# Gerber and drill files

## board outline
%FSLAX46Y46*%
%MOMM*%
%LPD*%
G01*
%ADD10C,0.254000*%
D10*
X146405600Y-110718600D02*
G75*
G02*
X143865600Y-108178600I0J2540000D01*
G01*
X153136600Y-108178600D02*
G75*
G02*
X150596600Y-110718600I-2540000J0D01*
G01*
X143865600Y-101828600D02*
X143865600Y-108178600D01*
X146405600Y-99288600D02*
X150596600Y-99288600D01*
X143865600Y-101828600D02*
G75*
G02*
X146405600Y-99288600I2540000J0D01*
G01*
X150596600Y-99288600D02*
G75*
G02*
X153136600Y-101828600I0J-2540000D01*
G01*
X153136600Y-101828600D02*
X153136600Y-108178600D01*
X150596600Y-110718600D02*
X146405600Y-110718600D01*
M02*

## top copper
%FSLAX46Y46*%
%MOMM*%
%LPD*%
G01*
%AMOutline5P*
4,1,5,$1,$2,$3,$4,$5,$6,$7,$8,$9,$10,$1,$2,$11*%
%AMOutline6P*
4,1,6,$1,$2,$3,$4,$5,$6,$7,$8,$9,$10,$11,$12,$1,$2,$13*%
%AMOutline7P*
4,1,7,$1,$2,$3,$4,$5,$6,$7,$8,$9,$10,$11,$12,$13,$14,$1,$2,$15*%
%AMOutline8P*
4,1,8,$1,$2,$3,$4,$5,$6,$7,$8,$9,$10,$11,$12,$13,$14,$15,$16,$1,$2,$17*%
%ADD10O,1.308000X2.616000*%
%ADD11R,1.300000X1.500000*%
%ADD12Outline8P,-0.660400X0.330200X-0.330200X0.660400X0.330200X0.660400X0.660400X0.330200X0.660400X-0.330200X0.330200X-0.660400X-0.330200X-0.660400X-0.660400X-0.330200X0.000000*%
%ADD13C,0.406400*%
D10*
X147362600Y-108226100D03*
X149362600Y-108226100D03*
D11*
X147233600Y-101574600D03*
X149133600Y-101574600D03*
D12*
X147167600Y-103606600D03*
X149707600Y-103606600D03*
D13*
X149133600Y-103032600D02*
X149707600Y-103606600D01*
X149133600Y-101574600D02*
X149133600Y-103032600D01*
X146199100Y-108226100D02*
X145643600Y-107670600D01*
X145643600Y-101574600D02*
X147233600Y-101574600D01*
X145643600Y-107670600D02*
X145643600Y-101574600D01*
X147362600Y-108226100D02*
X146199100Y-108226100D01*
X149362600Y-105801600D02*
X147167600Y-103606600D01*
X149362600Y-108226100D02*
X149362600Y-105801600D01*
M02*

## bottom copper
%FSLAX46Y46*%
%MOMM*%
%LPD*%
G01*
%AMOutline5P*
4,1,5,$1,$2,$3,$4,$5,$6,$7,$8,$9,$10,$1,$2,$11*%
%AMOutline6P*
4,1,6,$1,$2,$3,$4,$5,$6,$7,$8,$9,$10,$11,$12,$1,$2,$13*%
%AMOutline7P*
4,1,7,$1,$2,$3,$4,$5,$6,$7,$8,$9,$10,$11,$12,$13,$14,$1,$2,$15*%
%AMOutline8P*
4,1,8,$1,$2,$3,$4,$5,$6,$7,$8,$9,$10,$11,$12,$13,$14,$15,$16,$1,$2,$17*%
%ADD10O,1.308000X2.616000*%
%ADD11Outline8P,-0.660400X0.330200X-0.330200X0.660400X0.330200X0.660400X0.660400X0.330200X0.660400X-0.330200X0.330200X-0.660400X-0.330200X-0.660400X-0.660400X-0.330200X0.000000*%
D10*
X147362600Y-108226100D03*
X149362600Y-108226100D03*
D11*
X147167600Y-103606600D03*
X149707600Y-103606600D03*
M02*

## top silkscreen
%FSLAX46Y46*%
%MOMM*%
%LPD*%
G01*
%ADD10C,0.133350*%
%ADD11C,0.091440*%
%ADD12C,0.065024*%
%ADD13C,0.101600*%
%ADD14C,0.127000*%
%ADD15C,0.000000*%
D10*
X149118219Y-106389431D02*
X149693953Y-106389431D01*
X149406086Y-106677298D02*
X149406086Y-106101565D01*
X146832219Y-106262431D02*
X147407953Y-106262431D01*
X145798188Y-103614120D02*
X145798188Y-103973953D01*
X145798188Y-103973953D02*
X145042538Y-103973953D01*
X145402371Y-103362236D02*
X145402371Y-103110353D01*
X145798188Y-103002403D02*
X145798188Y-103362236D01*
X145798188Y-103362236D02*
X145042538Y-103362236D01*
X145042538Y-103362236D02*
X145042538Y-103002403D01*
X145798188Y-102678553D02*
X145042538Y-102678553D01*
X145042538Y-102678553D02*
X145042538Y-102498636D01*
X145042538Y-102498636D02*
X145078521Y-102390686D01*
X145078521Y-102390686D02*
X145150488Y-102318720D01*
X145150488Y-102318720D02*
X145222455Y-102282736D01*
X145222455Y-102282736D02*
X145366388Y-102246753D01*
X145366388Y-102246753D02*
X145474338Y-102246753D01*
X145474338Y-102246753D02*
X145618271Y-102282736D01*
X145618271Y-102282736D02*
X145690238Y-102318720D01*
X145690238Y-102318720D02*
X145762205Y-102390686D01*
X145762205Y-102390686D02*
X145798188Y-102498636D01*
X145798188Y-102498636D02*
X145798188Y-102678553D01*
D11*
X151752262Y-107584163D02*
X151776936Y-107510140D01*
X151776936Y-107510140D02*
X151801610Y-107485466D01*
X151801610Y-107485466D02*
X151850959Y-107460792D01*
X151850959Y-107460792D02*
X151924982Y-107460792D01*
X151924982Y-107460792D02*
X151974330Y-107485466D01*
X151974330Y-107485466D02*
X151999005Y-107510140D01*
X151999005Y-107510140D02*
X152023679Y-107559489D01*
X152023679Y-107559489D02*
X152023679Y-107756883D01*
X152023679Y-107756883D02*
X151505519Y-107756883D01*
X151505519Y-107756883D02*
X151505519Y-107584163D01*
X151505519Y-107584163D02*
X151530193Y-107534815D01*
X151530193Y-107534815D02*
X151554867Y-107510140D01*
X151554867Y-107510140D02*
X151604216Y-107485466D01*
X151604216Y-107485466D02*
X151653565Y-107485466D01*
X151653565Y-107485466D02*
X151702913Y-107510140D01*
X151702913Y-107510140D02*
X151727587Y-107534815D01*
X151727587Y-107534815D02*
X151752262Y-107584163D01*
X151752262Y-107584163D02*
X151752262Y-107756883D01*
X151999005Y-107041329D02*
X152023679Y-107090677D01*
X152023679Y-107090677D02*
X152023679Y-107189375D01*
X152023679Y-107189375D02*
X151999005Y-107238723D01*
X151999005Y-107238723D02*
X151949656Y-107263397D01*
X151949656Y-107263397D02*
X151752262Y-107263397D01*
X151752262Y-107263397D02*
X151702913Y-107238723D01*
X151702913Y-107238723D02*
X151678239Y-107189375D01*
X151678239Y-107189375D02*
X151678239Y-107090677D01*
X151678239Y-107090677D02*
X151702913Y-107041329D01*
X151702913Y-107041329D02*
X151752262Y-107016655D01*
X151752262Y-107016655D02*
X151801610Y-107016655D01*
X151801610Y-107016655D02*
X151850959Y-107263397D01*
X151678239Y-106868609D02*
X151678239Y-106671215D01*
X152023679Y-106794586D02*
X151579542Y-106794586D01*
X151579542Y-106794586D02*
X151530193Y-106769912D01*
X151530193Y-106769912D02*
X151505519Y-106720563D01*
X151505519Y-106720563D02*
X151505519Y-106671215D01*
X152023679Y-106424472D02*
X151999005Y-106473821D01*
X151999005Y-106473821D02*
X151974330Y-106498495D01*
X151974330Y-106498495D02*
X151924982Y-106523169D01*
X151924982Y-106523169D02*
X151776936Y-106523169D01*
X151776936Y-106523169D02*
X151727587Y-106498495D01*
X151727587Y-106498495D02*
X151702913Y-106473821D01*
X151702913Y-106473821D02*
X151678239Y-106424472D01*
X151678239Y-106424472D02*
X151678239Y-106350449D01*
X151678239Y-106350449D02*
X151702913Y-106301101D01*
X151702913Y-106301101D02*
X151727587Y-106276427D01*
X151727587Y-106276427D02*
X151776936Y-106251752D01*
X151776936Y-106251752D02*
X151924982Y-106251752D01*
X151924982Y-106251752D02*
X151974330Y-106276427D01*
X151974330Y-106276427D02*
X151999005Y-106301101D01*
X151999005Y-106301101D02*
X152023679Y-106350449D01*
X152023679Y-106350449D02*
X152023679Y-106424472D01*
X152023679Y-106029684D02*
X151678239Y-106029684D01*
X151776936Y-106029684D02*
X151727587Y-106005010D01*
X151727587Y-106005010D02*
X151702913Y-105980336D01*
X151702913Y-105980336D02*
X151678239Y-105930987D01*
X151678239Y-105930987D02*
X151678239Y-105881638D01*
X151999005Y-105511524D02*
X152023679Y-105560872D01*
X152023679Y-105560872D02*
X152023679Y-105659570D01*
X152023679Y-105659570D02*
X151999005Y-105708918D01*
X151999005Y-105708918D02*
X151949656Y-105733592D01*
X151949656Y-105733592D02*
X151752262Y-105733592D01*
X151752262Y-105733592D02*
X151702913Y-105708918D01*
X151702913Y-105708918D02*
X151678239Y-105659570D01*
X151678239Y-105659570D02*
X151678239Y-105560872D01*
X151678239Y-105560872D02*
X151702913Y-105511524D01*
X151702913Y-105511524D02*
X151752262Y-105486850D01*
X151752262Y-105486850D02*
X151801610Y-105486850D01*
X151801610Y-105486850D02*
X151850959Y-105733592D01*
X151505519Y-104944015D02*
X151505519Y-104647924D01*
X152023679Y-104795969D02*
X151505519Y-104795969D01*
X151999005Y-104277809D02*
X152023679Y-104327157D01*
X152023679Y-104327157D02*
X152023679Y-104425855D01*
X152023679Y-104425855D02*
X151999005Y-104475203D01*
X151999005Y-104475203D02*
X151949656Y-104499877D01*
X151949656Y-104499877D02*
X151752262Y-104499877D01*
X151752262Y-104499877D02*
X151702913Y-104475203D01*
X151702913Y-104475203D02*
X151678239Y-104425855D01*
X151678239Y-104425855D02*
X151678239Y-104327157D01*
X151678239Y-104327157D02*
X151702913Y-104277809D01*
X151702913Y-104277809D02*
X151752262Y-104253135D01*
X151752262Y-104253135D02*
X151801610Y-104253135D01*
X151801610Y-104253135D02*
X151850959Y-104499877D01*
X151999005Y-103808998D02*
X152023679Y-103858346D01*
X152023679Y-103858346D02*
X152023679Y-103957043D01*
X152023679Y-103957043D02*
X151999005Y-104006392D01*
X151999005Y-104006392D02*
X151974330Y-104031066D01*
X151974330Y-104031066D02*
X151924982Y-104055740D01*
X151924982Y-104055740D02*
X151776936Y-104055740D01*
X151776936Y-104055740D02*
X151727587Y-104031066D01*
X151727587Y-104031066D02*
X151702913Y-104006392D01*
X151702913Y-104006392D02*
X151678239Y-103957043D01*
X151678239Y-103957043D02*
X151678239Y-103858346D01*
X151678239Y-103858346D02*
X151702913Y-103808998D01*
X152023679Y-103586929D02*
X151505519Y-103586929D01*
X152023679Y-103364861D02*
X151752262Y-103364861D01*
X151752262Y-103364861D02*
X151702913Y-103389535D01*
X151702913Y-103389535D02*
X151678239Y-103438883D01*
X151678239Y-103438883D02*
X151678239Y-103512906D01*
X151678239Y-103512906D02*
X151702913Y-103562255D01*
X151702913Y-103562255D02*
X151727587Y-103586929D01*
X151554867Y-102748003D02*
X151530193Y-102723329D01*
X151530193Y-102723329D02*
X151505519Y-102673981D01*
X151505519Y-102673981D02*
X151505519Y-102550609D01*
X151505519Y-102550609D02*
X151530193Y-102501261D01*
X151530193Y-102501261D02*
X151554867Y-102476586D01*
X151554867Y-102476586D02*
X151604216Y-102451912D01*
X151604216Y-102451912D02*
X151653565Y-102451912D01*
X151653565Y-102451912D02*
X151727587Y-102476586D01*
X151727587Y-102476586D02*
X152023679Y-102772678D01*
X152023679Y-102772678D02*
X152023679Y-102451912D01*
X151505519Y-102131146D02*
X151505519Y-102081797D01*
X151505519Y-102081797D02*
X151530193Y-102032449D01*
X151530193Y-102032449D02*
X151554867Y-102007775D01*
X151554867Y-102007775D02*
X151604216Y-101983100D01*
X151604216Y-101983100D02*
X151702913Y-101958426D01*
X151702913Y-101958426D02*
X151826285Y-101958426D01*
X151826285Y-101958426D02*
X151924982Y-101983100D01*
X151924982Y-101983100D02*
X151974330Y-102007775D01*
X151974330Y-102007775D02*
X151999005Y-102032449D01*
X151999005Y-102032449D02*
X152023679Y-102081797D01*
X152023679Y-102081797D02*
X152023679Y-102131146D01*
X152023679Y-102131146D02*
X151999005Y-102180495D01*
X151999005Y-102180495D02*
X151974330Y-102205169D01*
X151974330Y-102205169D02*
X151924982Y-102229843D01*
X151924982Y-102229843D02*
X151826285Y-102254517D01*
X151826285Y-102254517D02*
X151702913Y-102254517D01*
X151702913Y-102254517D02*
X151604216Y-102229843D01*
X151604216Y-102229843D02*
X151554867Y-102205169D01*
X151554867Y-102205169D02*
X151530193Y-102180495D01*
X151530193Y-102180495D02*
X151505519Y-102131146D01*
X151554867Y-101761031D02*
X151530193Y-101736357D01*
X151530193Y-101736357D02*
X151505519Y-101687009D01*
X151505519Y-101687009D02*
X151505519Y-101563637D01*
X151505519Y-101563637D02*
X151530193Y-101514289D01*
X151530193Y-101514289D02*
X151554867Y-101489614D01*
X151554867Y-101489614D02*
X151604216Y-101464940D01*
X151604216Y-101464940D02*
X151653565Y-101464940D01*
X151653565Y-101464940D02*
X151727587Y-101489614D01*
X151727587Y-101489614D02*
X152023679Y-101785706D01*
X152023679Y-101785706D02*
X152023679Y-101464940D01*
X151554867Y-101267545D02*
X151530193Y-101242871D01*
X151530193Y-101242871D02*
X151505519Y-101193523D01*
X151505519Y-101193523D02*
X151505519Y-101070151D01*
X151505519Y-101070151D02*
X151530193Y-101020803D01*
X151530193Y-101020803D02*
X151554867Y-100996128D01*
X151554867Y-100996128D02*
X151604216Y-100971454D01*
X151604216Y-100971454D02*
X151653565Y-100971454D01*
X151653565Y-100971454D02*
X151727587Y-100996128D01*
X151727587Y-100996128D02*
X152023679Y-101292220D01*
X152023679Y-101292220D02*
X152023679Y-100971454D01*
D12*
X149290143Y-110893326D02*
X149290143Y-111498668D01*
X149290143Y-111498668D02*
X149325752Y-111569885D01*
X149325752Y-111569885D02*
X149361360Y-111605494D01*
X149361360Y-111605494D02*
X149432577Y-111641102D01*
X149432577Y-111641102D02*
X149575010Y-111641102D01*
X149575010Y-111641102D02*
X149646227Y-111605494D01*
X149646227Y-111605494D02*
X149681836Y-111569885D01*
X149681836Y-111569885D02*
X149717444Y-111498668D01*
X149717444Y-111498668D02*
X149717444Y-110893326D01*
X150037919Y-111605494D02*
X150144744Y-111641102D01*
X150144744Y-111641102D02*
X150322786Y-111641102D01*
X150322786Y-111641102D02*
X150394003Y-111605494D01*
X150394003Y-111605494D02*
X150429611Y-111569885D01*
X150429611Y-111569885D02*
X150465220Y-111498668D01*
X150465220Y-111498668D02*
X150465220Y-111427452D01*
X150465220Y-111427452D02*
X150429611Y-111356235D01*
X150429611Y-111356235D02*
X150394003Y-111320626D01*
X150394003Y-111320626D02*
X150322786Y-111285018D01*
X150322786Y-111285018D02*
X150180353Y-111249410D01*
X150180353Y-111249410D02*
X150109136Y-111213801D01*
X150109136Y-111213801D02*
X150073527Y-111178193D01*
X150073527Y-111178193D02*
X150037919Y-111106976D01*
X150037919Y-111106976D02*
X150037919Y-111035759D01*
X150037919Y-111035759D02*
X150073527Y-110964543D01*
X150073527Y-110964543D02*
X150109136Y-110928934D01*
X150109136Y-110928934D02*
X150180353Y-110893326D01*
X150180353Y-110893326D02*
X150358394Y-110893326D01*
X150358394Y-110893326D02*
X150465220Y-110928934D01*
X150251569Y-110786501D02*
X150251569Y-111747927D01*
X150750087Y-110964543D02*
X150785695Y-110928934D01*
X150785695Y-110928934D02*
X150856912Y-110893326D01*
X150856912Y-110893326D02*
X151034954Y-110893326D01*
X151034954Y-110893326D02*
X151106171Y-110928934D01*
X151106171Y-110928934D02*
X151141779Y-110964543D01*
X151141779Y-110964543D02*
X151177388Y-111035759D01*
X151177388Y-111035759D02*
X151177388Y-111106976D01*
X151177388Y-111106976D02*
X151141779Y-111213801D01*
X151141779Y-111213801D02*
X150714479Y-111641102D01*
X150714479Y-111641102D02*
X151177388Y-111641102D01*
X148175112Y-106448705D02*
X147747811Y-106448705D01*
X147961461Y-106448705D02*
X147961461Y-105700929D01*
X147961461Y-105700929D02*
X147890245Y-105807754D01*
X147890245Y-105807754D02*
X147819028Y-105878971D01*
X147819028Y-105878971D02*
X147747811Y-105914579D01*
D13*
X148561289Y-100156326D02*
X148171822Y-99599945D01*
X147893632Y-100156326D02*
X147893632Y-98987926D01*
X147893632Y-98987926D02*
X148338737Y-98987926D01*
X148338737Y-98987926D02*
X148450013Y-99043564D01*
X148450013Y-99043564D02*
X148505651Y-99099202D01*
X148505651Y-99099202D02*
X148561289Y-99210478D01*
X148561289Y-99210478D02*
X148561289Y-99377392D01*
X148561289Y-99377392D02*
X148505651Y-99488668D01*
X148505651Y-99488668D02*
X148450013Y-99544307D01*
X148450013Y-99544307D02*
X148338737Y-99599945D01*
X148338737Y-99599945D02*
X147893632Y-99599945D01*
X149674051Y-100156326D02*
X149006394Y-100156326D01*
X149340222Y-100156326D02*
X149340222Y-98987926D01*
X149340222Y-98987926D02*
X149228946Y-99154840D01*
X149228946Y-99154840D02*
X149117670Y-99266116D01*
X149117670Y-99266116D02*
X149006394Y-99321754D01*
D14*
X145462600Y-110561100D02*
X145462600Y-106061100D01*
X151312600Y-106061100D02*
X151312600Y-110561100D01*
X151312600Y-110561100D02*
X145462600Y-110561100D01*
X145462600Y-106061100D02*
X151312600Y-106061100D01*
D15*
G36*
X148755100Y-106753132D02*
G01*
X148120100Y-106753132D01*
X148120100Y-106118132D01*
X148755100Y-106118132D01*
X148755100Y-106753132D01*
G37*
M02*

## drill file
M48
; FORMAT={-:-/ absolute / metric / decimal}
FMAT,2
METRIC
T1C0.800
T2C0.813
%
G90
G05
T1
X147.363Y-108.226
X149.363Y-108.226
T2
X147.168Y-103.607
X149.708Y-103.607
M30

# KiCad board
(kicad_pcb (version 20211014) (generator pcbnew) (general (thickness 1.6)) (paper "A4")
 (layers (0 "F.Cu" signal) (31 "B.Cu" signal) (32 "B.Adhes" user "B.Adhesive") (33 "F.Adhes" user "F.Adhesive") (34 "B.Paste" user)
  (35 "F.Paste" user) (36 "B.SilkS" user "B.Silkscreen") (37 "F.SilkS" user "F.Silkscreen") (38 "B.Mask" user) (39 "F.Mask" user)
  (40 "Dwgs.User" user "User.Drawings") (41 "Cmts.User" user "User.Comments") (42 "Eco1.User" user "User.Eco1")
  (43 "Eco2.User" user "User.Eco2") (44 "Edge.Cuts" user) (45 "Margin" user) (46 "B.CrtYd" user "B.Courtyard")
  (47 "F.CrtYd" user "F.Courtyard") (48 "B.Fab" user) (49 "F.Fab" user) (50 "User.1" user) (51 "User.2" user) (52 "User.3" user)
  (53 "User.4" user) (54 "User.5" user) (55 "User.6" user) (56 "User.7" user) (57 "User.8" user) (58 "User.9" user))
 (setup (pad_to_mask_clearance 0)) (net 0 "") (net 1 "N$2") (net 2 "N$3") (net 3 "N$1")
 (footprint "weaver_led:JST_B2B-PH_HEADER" (layer "F.Cu") (at 148.4376 108.1786 180)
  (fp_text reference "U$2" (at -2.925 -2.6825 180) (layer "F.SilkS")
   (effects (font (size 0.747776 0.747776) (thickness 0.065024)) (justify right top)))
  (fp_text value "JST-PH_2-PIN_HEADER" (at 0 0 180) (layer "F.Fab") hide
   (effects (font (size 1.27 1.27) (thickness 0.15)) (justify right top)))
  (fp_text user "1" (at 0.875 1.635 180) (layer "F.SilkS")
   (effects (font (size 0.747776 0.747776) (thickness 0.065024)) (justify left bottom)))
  (fp_line (start 2.975 -2.3825) (end 2.975 2.1175) (layer "F.SilkS") (width 0.127))
  (fp_line (start -2.875 2.1175) (end -2.875 -2.3825) (layer "F.SilkS") (width 0.127))
  (fp_line (start -2.875 -2.3825) (end 2.975 -2.3825) (layer "F.SilkS") (width 0.127))
  (fp_line (start 2.975 2.1175) (end -2.875 2.1175) (layer "F.SilkS") (width 0.127))
  (fp_poly
   (pts (xy -0.3175 2.060468) (xy 0.3175 2.060468) (xy 0.3175 1.425468) (xy -0.3175 1.425468)) (layer "F.SilkS") (width 0) (fill solid))
  (pad "P1" thru_hole oval (at 1.075 -0.0475 270) (size 2.616 1.308) (drill 0.8) (layers *.Cu *.Mask) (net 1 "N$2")
   (solder_mask_margin 0.1016))
  (pad "P2" thru_hole oval (at -0.925 -0.0475 270) (size 2.616 1.308) (drill 0.8) (layers *.Cu *.Mask) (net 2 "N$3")
   (solder_mask_margin 0.1016)))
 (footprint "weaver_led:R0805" (layer "F.Cu") (at 148.1836 101.5746)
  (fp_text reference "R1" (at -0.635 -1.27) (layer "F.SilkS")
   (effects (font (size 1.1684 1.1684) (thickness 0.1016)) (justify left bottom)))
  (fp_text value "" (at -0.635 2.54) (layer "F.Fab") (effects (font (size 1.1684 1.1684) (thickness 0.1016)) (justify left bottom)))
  (pad "1" smd rect (at -0.95 0) (size 1.3 1.5) (layers "F.Cu" "F.Paste" "F.Mask") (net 1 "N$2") (solder_mask_margin 0.1016))
  (pad "2" smd rect (at 0.95 0) (size 1.3 1.5) (layers "F.Cu" "F.Paste" "F.Mask") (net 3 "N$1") (solder_mask_margin 0.1016)))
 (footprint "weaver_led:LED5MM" (layer "B.Cu") (at 148.4376 103.6066)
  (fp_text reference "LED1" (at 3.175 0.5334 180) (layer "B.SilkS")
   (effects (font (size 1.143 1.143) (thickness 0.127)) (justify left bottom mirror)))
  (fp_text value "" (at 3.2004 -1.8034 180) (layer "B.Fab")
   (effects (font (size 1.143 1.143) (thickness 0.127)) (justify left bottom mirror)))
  (pad "A" thru_hole roundrect (at -1.27 0) (size 1.3208 1.3208) (drill 0.8128) (layers *.Cu *.Mask) (roundrect_rratio 0.25)
   (chamfer_ratio 0.25) (chamfer top_left top_right bottom_left bottom_right) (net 2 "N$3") (solder_mask_margin 0.1016))
  (pad "K" thru_hole roundrect (at 1.27 0) (size 1.3208 1.3208) (drill 0.8128) (layers *.Cu *.Mask) (roundrect_rratio 0.25)
   (chamfer_ratio 0.25) (chamfer top_left top_right bottom_left bottom_right) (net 3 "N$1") (solder_mask_margin 0.1016)))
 (gr_arc (start 146.4056 110.7186) (mid 144.609549 109.974651) (end 143.8656 108.1786) (layer "Edge.Cuts") (width 0.254))
 (gr_arc (start 153.1366 108.1786) (mid 152.392651 109.974651) (end 150.5966 110.7186) (layer "Edge.Cuts") (width 0.254))
 (gr_line (start 143.8656 101.8286) (end 143.8656 108.1786) (layer "Edge.Cuts") (width 0.254))
 (gr_line (start 146.4056 99.2886) (end 150.5966 99.2886) (layer "Edge.Cuts") (width 0.254))
 (gr_arc (start 143.8656 101.8286) (mid 144.609549 100.032549) (end 146.4056 99.2886) (layer "Edge.Cuts") (width 0.254))
 (gr_arc (start 150.5966 99.2886) (mid 152.392651 100.032549) (end 153.1366 101.8286) (layer "Edge.Cuts") (width 0.254))
 (gr_line (start 153.1366 101.8286) (end 153.1366 108.1786) (layer "Edge.Cuts") (width 0.254))
 (gr_line (start 150.5966 110.7186) (end 146.4056 110.7186) (layer "Edge.Cuts") (width 0.254))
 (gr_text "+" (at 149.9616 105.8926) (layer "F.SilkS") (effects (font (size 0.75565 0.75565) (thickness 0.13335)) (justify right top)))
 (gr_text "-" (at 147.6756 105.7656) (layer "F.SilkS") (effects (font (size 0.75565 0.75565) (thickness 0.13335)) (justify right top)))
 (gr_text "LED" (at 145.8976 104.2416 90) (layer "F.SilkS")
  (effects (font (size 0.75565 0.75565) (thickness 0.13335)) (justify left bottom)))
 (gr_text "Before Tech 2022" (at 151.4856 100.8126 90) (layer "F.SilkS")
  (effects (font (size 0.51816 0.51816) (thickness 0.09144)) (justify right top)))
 (segment (start 149.1336 103.0326) (end 149.7076 103.6066) (width 0.4064) (layer "F.Cu") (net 3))
 (segment (start 149.1336 101.5746) (end 149.1336 103.0326) (width 0.4064) (layer "F.Cu") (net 3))
 (segment (start 146.1991 108.2261) (end 145.6436 107.6706) (width 0.4064) (layer "F.Cu") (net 1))
 (segment (start 145.6436 101.5746) (end 147.2336 101.5746) (width 0.4064) (layer "F.Cu") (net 1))
 (segment (start 145.6436 107.6706) (end 145.6436 101.5746) (width 0.4064) (layer "F.Cu") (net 1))
 (segment (start 147.3626 108.2261) (end 146.1991 108.2261) (width 0.4064) (layer "F.Cu") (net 1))
 (segment (start 149.3626 105.8016) (end 147.1676 103.6066) (width 0.4064) (layer "F.Cu") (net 2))
 (segment (start 149.3626 108.2261) (end 149.3626 105.8016) (width 0.4064) (layer "F.Cu") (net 2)))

